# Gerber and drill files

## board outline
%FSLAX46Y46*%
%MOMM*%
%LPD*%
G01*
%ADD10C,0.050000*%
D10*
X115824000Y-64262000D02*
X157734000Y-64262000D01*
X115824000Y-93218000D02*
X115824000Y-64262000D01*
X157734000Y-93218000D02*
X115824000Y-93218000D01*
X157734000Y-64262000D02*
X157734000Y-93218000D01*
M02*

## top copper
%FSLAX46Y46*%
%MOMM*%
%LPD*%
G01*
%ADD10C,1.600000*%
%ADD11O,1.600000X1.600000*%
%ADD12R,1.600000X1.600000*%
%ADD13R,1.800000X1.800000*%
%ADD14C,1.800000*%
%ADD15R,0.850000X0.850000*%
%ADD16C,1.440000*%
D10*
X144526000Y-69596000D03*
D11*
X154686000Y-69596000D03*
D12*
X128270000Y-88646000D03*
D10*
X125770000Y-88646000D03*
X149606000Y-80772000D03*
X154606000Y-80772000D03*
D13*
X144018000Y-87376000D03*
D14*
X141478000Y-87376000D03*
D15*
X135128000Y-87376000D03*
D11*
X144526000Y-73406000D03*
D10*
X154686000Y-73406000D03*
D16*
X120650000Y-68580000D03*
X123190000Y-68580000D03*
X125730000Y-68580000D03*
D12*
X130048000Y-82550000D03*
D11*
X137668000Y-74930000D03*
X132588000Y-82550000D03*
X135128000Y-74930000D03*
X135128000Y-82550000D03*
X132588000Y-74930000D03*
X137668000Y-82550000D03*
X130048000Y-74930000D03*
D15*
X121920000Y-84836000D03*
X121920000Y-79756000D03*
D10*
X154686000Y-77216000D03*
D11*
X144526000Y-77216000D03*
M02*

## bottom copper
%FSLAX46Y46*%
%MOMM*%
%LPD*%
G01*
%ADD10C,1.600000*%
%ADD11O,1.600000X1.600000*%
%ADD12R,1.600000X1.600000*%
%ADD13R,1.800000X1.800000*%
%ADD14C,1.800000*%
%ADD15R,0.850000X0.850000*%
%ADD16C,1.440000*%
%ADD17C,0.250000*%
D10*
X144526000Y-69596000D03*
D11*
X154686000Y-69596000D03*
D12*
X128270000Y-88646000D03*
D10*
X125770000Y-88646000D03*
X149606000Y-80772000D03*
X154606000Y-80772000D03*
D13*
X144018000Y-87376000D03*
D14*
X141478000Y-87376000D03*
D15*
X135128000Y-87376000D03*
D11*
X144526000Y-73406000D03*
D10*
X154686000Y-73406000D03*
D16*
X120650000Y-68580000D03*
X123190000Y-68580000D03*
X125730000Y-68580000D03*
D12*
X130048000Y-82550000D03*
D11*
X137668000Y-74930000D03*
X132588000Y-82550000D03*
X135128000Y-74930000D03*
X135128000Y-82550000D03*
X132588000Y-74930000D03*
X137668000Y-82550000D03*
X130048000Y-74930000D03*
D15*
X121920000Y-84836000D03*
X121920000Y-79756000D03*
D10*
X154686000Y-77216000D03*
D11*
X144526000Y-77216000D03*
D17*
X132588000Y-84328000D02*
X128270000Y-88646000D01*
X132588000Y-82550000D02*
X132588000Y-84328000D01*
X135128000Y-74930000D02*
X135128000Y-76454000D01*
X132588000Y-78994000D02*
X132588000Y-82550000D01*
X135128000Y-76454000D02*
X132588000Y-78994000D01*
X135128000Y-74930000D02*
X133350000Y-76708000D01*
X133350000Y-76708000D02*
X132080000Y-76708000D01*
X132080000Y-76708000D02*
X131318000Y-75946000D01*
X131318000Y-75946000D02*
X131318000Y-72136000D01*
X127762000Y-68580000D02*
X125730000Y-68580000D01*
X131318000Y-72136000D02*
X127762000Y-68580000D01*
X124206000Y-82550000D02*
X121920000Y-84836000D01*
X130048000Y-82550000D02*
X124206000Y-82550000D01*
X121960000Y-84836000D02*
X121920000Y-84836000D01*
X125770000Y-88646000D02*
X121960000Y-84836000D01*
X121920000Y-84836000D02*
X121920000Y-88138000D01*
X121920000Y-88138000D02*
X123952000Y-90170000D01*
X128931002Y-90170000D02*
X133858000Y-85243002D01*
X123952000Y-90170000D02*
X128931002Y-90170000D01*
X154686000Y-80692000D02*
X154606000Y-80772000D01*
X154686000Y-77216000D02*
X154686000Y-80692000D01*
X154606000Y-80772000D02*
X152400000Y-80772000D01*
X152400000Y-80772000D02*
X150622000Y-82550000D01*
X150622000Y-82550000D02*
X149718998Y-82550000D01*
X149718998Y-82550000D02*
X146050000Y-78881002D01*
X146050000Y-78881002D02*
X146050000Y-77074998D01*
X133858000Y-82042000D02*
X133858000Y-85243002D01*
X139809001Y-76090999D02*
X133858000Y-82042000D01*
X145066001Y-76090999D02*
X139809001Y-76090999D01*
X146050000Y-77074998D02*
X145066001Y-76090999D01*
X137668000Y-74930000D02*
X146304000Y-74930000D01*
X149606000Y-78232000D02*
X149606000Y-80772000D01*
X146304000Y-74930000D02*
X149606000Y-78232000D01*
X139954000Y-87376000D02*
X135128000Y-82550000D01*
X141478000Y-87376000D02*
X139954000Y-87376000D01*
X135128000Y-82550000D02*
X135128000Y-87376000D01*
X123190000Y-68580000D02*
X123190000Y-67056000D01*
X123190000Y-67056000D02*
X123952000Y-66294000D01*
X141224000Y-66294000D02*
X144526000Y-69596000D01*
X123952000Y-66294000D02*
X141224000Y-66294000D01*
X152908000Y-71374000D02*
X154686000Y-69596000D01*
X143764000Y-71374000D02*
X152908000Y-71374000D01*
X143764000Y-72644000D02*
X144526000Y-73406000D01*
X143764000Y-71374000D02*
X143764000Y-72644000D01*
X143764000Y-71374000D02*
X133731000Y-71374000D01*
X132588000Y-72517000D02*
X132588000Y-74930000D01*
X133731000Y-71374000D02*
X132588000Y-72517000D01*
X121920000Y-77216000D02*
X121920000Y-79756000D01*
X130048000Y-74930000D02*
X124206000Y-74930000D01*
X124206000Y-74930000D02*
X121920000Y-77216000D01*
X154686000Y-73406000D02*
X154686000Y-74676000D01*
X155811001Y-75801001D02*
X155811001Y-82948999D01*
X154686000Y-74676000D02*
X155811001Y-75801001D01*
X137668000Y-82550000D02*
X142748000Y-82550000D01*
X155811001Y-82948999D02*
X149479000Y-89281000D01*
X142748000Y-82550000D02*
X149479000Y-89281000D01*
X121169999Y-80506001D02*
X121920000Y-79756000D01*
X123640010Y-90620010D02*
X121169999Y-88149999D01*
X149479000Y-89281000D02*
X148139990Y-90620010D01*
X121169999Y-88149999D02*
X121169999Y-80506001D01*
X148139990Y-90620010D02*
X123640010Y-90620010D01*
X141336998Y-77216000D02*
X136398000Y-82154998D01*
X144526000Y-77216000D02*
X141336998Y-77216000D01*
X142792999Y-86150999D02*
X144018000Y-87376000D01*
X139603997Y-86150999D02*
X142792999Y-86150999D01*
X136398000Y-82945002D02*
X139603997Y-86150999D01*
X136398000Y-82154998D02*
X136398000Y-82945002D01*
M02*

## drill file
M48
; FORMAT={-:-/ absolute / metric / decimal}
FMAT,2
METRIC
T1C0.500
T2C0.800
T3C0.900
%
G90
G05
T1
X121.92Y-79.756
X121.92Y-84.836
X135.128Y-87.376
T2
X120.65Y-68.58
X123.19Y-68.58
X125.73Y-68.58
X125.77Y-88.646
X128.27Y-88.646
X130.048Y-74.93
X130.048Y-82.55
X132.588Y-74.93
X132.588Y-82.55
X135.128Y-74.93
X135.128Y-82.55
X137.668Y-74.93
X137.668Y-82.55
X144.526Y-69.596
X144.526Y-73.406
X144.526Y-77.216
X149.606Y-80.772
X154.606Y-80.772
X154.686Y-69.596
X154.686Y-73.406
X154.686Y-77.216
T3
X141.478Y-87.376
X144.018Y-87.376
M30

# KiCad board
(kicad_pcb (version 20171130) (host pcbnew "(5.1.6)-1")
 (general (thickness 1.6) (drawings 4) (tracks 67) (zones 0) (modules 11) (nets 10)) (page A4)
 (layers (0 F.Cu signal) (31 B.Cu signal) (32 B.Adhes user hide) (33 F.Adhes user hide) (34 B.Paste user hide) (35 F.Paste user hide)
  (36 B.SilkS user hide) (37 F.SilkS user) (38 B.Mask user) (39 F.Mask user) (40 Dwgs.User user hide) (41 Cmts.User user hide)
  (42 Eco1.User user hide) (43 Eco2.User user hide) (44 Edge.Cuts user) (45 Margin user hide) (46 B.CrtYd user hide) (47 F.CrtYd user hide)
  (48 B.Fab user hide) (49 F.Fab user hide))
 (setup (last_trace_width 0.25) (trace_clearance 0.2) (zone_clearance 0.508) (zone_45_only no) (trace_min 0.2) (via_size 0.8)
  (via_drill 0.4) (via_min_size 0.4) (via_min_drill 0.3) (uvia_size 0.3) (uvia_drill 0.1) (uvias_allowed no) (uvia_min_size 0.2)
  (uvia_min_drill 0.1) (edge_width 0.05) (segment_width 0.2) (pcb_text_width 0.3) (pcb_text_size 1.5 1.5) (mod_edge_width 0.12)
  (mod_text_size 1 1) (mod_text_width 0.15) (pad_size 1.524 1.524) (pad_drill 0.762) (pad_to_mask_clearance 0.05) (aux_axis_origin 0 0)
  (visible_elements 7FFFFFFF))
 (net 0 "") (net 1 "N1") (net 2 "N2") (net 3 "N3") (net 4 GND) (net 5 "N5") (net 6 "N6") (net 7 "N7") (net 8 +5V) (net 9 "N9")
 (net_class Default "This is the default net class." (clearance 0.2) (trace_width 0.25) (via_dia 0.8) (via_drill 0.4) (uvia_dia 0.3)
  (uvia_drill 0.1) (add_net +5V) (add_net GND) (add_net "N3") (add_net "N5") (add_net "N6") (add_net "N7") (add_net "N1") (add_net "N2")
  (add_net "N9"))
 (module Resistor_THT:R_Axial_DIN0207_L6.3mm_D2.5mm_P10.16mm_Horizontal (layer F.Cu) (at 144.526 69.596)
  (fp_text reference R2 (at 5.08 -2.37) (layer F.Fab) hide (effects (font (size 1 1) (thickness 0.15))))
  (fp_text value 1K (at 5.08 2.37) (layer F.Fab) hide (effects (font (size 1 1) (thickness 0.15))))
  (pad 1 thru_hole circle (at 0 0) (size 1.6 1.6) (drill 0.8) (layers *.Cu *.Mask) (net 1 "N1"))
  (pad 2 thru_hole oval (at 10.16 0) (size 1.6 1.6) (drill 0.8) (layers *.Cu *.Mask) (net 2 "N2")))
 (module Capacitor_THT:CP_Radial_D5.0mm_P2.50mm (layer F.Cu) (at 128.27 88.646 180)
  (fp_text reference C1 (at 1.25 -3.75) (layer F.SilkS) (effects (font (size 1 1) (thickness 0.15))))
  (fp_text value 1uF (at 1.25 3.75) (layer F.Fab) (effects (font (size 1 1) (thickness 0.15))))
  (pad 1 thru_hole rect (at 0 0 180) (size 1.6 1.6) (drill 0.8) (layers *.Cu *.Mask) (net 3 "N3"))
  (pad 2 thru_hole circle (at 2.5 0 180) (size 1.6 1.6) (drill 0.8) (layers *.Cu *.Mask) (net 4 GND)))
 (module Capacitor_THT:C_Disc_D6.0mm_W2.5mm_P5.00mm (layer F.Cu) (at 149.606 80.772)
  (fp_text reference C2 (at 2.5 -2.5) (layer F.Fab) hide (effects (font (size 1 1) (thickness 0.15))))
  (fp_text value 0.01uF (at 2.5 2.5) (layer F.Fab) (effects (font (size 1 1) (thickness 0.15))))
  (pad 1 thru_hole circle (at 0 0) (size 1.6 1.6) (drill 0.8) (layers *.Cu *.Mask) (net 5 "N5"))
  (pad 2 thru_hole circle (at 5 0) (size 1.6 1.6) (drill 0.8) (layers *.Cu *.Mask) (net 4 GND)))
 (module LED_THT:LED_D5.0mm (layer F.Cu) (at 144.018 87.376 180)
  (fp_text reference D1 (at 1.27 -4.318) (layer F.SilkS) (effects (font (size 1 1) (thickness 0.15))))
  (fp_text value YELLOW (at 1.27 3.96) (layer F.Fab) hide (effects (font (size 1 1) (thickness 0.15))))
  (pad 1 thru_hole rect (at 0 0 180) (size 1.8 1.8) (drill 0.9) (layers *.Cu *.Mask) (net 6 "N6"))
  (pad 2 thru_hole circle (at 2.54 0 180) (size 1.8 1.8) (drill 0.9) (layers *.Cu *.Mask) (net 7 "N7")))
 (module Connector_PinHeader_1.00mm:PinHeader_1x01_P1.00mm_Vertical (layer F.Cu) (at 135.128 87.376)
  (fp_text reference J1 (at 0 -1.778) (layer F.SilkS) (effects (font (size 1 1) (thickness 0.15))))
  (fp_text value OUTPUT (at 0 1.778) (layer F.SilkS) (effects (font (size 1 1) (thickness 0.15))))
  (pad 1 thru_hole rect (at 0 0) (size 0.85 0.85) (drill 0.5) (layers *.Cu *.Mask) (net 7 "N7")))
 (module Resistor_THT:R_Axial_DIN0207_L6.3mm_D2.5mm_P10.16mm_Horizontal (layer F.Cu) (at 154.686 73.406 180)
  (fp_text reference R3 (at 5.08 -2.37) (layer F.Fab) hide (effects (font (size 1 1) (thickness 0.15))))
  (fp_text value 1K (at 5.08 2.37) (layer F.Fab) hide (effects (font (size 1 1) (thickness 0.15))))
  (pad 2 thru_hole oval (at 10.16 0 180) (size 1.6 1.6) (drill 0.8) (layers *.Cu *.Mask) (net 2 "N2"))
  (pad 1 thru_hole circle (at 0 0 180) (size 1.6 1.6) (drill 0.8) (layers *.Cu *.Mask) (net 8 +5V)))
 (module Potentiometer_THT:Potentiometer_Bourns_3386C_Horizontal (layer F.Cu) (at 125.73 68.58 270)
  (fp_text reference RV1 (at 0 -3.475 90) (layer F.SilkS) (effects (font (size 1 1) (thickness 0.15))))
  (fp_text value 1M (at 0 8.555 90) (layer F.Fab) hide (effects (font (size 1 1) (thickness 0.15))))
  (pad 3 thru_hole circle (at 0 5.08 270) (size 1.44 1.44) (drill 0.8) (layers *.Cu *.Mask) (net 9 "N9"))
  (pad 2 thru_hole circle (at 0 2.54 270) (size 1.44 1.44) (drill 0.8) (layers *.Cu *.Mask) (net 1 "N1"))
  (pad 1 thru_hole circle (at 0 0 270) (size 1.44 1.44) (drill 0.8) (layers *.Cu *.Mask) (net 3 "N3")))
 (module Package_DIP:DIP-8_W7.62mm (layer F.Cu) (at 130.048 82.55 90)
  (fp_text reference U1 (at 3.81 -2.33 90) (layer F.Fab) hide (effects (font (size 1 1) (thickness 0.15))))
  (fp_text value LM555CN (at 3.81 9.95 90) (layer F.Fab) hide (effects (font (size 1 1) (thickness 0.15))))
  (pad 1 thru_hole rect (at 0 0 90) (size 1.6 1.6) (drill 0.8) (layers *.Cu *.Mask) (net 4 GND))
  (pad 5 thru_hole oval (at 7.62 7.62 90) (size 1.6 1.6) (drill 0.8) (layers *.Cu *.Mask) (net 5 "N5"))
  (pad 2 thru_hole oval (at 0 2.54 90) (size 1.6 1.6) (drill 0.8) (layers *.Cu *.Mask) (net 3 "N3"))
  (pad 6 thru_hole oval (at 7.62 5.08 90) (size 1.6 1.6) (drill 0.8) (layers *.Cu *.Mask) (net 3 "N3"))
  (pad 3 thru_hole oval (at 0 5.08 90) (size 1.6 1.6) (drill 0.8) (layers *.Cu *.Mask) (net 7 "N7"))
  (pad 7 thru_hole oval (at 7.62 2.54 90) (size 1.6 1.6) (drill 0.8) (layers *.Cu *.Mask) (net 2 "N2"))
  (pad 4 thru_hole oval (at 0 7.62 90) (size 1.6 1.6) (drill 0.8) (layers *.Cu *.Mask) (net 8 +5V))
  (pad 8 thru_hole oval (at 7.62 0 90) (size 1.6 1.6) (drill 0.8) (layers *.Cu *.Mask) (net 8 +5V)))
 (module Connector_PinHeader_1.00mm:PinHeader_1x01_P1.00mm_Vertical (layer F.Cu) (at 121.92 84.836)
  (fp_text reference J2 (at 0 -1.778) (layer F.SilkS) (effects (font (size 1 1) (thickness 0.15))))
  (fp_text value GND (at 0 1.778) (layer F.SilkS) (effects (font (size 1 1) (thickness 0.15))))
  (pad 1 thru_hole rect (at 0 0) (size 0.85 0.85) (drill 0.5) (layers *.Cu *.Mask) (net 4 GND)))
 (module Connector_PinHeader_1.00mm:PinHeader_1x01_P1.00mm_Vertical (layer F.Cu) (at 121.92 79.756)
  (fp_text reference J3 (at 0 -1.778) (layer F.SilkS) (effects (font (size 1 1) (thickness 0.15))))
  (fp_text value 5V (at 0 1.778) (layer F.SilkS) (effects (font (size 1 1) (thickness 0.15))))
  (pad 1 thru_hole rect (at 0 0) (size 0.85 0.85) (drill 0.5) (layers *.Cu *.Mask) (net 8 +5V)))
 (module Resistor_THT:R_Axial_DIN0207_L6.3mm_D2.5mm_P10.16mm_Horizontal (layer F.Cu) (at 154.686 77.216 180)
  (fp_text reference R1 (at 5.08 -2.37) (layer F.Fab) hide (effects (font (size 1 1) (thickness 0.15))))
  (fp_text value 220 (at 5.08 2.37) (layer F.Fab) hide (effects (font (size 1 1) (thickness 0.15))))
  (pad 1 thru_hole circle (at 0 0 180) (size 1.6 1.6) (drill 0.8) (layers *.Cu *.Mask) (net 4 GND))
  (pad 2 thru_hole oval (at 10.16 0 180) (size 1.6 1.6) (drill 0.8) (layers *.Cu *.Mask) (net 6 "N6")))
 (gr_line (start 115.824 64.262) (end 157.734 64.262) (layer Edge.Cuts) (width 0.05))
 (gr_line (start 115.824 93.218) (end 115.824 64.262) (layer Edge.Cuts) (width 0.05))
 (gr_line (start 157.734 93.218) (end 115.824 93.218) (layer Edge.Cuts) (width 0.05))
 (gr_line (start 157.734 64.262) (end 157.734 93.218) (layer Edge.Cuts) (width 0.05))
 (segment (start 132.588 84.328) (end 128.27 88.646) (width 0.25) (layer B.Cu) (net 3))
 (segment (start 132.588 82.55) (end 132.588 84.328) (width 0.25) (layer B.Cu) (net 3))
 (segment (start 135.128 74.93) (end 135.128 76.454) (width 0.25) (layer B.Cu) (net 3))
 (segment (start 132.588 78.994) (end 132.588 82.55) (width 0.25) (layer B.Cu) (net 3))
 (segment (start 135.128 76.454) (end 132.588 78.994) (width 0.25) (layer B.Cu) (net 3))
 (segment (start 135.128 74.93) (end 133.35 76.708) (width 0.25) (layer B.Cu) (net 3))
 (segment (start 133.35 76.708) (end 132.08 76.708) (width 0.25) (layer B.Cu) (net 3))
 (segment (start 132.08 76.708) (end 131.318 75.946) (width 0.25) (layer B.Cu) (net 3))
 (segment (start 131.318 75.946) (end 131.318 72.136) (width 0.25) (layer B.Cu) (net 3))
 (segment (start 127.762 68.58) (end 125.73 68.58) (width 0.25) (layer B.Cu) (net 3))
 (segment (start 131.318 72.136) (end 127.762 68.58) (width 0.25) (layer B.Cu) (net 3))
 (segment (start 124.206 82.55) (end 121.92 84.836) (width 0.25) (layer B.Cu) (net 4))
 (segment (start 130.048 82.55) (end 124.206 82.55) (width 0.25) (layer B.Cu) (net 4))
 (segment (start 121.96 84.836) (end 121.92 84.836) (width 0.25) (layer B.Cu) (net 4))
 (segment (start 125.77 88.646) (end 121.96 84.836) (width 0.25) (layer B.Cu) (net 4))
 (segment (start 121.92 84.836) (end 121.92 88.138) (width 0.25) (layer B.Cu) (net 4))
 (segment (start 121.92 88.138) (end 123.952 90.17) (width 0.25) (layer B.Cu) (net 4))
 (segment (start 128.931002 90.17) (end 133.858 85.243002) (width 0.25) (layer B.Cu) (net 4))
 (segment (start 123.952 90.17) (end 128.931002 90.17) (width 0.25) (layer B.Cu) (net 4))
 (segment (start 154.686 80.692) (end 154.606 80.772) (width 0.25) (layer B.Cu) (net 4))
 (segment (start 154.686 77.216) (end 154.686 80.692) (width 0.25) (layer B.Cu) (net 4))
 (segment (start 154.606 80.772) (end 152.4 80.772) (width 0.25) (layer B.Cu) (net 4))
 (segment (start 152.4 80.772) (end 150.622 82.55) (width 0.25) (layer B.Cu) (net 4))
 (segment (start 150.622 82.55) (end 149.718998 82.55) (width 0.25) (layer B.Cu) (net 4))
 (segment (start 149.718998 82.55) (end 146.05 78.881002) (width 0.25) (layer B.Cu) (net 4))
 (segment (start 146.05 78.881002) (end 146.05 77.074998) (width 0.25) (layer B.Cu) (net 4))
 (segment (start 133.858 82.042) (end 133.858 85.243002) (width 0.25) (layer B.Cu) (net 4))
 (segment (start 139.809001 76.090999) (end 133.858 82.042) (width 0.25) (layer B.Cu) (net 4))
 (segment (start 145.066001 76.090999) (end 139.809001 76.090999) (width 0.25) (layer B.Cu) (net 4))
 (segment (start 146.05 77.074998) (end 145.066001 76.090999) (width 0.25) (layer B.Cu) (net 4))
 (segment (start 137.668 74.93) (end 146.304 74.93) (width 0.25) (layer B.Cu) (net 5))
 (segment (start 149.606 78.232) (end 149.606 80.772) (width 0.25) (layer B.Cu) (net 5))
 (segment (start 146.304 74.93) (end 149.606 78.232) (width 0.25) (layer B.Cu) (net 5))
 (segment (start 139.954 87.376) (end 135.128 82.55) (width 0.25) (layer B.Cu) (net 7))
 (segment (start 141.478 87.376) (end 139.954 87.376) (width 0.25) (layer B.Cu) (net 7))
 (segment (start 135.128 82.55) (end 135.128 87.376) (width 0.25) (layer B.Cu) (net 7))
 (segment (start 123.19 68.58) (end 123.19 67.056) (width 0.25) (layer B.Cu) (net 1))
 (segment (start 123.19 67.056) (end 123.952 66.294) (width 0.25) (layer B.Cu) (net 1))
 (segment (start 141.224 66.294) (end 144.526 69.596) (width 0.25) (layer B.Cu) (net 1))
 (segment (start 123.952 66.294) (end 141.224 66.294) (width 0.25) (layer B.Cu) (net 1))
 (segment (start 152.908 71.374) (end 154.686 69.596) (width 0.25) (layer B.Cu) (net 2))
 (segment (start 143.764 71.374) (end 152.908 71.374) (width 0.25) (layer B.Cu) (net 2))
 (segment (start 143.764 72.644) (end 144.526 73.406) (width 0.25) (layer B.Cu) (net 2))
 (segment (start 143.764 71.374) (end 143.764 72.644) (width 0.25) (layer B.Cu) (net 2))
 (segment (start 143.764 71.374) (end 133.731 71.374) (width 0.25) (layer B.Cu) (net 2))
 (segment (start 132.588 72.517) (end 132.588 74.93) (width 0.25) (layer B.Cu) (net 2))
 (segment (start 133.731 71.374) (end 132.588 72.517) (width 0.25) (layer B.Cu) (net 2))
 (segment (start 121.92 77.216) (end 121.92 79.756) (width 0.25) (layer B.Cu) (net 8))
 (segment (start 130.048 74.93) (end 124.206 74.93) (width 0.25) (layer B.Cu) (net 8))
 (segment (start 124.206 74.93) (end 121.92 77.216) (width 0.25) (layer B.Cu) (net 8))
 (segment (start 154.686 73.406) (end 154.686 74.676) (width 0.25) (layer B.Cu) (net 8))
 (segment (start 155.811001 75.801001) (end 155.811001 82.948999) (width 0.25) (layer B.Cu) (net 8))
 (segment (start 154.686 74.676) (end 155.811001 75.801001) (width 0.25) (layer B.Cu) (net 8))
 (segment (start 137.668 82.55) (end 142.748 82.55) (width 0.25) (layer B.Cu) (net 8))
 (segment (start 155.811001 82.948999) (end 149.479 89.281) (width 0.25) (layer B.Cu) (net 8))
 (segment (start 142.748 82.55) (end 149.479 89.281) (width 0.25) (layer B.Cu) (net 8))
 (segment (start 121.169999 80.506001) (end 121.92 79.756) (width 0.25) (layer B.Cu) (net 8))
 (segment (start 123.64001 90.62001) (end 121.169999 88.149999) (width 0.25) (layer B.Cu) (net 8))
 (segment (start 149.479 89.281) (end 148.13999 90.62001) (width 0.25) (layer B.Cu) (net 8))
 (segment (start 121.169999 88.149999) (end 121.169999 80.506001) (width 0.25) (layer B.Cu) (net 8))
 (segment (start 148.13999 90.62001) (end 123.64001 90.62001) (width 0.25) (layer B.Cu) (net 8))
 (segment (start 141.336998 77.216) (end 136.398 82.154998) (width 0.25) (layer B.Cu) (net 6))
 (segment (start 144.526 77.216) (end 141.336998 77.216) (width 0.25) (layer B.Cu) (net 6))
 (segment (start 142.792999 86.150999) (end 144.018 87.376) (width 0.25) (layer B.Cu) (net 6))
 (segment (start 139.603997 86.150999) (end 142.792999 86.150999) (width 0.25) (layer B.Cu) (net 6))
 (segment (start 136.398 82.945002) (end 139.603997 86.150999) (width 0.25) (layer B.Cu) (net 6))
 (segment (start 136.398 82.154998) (end 136.398 82.945002) (width 0.25) (layer B.Cu) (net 6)))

